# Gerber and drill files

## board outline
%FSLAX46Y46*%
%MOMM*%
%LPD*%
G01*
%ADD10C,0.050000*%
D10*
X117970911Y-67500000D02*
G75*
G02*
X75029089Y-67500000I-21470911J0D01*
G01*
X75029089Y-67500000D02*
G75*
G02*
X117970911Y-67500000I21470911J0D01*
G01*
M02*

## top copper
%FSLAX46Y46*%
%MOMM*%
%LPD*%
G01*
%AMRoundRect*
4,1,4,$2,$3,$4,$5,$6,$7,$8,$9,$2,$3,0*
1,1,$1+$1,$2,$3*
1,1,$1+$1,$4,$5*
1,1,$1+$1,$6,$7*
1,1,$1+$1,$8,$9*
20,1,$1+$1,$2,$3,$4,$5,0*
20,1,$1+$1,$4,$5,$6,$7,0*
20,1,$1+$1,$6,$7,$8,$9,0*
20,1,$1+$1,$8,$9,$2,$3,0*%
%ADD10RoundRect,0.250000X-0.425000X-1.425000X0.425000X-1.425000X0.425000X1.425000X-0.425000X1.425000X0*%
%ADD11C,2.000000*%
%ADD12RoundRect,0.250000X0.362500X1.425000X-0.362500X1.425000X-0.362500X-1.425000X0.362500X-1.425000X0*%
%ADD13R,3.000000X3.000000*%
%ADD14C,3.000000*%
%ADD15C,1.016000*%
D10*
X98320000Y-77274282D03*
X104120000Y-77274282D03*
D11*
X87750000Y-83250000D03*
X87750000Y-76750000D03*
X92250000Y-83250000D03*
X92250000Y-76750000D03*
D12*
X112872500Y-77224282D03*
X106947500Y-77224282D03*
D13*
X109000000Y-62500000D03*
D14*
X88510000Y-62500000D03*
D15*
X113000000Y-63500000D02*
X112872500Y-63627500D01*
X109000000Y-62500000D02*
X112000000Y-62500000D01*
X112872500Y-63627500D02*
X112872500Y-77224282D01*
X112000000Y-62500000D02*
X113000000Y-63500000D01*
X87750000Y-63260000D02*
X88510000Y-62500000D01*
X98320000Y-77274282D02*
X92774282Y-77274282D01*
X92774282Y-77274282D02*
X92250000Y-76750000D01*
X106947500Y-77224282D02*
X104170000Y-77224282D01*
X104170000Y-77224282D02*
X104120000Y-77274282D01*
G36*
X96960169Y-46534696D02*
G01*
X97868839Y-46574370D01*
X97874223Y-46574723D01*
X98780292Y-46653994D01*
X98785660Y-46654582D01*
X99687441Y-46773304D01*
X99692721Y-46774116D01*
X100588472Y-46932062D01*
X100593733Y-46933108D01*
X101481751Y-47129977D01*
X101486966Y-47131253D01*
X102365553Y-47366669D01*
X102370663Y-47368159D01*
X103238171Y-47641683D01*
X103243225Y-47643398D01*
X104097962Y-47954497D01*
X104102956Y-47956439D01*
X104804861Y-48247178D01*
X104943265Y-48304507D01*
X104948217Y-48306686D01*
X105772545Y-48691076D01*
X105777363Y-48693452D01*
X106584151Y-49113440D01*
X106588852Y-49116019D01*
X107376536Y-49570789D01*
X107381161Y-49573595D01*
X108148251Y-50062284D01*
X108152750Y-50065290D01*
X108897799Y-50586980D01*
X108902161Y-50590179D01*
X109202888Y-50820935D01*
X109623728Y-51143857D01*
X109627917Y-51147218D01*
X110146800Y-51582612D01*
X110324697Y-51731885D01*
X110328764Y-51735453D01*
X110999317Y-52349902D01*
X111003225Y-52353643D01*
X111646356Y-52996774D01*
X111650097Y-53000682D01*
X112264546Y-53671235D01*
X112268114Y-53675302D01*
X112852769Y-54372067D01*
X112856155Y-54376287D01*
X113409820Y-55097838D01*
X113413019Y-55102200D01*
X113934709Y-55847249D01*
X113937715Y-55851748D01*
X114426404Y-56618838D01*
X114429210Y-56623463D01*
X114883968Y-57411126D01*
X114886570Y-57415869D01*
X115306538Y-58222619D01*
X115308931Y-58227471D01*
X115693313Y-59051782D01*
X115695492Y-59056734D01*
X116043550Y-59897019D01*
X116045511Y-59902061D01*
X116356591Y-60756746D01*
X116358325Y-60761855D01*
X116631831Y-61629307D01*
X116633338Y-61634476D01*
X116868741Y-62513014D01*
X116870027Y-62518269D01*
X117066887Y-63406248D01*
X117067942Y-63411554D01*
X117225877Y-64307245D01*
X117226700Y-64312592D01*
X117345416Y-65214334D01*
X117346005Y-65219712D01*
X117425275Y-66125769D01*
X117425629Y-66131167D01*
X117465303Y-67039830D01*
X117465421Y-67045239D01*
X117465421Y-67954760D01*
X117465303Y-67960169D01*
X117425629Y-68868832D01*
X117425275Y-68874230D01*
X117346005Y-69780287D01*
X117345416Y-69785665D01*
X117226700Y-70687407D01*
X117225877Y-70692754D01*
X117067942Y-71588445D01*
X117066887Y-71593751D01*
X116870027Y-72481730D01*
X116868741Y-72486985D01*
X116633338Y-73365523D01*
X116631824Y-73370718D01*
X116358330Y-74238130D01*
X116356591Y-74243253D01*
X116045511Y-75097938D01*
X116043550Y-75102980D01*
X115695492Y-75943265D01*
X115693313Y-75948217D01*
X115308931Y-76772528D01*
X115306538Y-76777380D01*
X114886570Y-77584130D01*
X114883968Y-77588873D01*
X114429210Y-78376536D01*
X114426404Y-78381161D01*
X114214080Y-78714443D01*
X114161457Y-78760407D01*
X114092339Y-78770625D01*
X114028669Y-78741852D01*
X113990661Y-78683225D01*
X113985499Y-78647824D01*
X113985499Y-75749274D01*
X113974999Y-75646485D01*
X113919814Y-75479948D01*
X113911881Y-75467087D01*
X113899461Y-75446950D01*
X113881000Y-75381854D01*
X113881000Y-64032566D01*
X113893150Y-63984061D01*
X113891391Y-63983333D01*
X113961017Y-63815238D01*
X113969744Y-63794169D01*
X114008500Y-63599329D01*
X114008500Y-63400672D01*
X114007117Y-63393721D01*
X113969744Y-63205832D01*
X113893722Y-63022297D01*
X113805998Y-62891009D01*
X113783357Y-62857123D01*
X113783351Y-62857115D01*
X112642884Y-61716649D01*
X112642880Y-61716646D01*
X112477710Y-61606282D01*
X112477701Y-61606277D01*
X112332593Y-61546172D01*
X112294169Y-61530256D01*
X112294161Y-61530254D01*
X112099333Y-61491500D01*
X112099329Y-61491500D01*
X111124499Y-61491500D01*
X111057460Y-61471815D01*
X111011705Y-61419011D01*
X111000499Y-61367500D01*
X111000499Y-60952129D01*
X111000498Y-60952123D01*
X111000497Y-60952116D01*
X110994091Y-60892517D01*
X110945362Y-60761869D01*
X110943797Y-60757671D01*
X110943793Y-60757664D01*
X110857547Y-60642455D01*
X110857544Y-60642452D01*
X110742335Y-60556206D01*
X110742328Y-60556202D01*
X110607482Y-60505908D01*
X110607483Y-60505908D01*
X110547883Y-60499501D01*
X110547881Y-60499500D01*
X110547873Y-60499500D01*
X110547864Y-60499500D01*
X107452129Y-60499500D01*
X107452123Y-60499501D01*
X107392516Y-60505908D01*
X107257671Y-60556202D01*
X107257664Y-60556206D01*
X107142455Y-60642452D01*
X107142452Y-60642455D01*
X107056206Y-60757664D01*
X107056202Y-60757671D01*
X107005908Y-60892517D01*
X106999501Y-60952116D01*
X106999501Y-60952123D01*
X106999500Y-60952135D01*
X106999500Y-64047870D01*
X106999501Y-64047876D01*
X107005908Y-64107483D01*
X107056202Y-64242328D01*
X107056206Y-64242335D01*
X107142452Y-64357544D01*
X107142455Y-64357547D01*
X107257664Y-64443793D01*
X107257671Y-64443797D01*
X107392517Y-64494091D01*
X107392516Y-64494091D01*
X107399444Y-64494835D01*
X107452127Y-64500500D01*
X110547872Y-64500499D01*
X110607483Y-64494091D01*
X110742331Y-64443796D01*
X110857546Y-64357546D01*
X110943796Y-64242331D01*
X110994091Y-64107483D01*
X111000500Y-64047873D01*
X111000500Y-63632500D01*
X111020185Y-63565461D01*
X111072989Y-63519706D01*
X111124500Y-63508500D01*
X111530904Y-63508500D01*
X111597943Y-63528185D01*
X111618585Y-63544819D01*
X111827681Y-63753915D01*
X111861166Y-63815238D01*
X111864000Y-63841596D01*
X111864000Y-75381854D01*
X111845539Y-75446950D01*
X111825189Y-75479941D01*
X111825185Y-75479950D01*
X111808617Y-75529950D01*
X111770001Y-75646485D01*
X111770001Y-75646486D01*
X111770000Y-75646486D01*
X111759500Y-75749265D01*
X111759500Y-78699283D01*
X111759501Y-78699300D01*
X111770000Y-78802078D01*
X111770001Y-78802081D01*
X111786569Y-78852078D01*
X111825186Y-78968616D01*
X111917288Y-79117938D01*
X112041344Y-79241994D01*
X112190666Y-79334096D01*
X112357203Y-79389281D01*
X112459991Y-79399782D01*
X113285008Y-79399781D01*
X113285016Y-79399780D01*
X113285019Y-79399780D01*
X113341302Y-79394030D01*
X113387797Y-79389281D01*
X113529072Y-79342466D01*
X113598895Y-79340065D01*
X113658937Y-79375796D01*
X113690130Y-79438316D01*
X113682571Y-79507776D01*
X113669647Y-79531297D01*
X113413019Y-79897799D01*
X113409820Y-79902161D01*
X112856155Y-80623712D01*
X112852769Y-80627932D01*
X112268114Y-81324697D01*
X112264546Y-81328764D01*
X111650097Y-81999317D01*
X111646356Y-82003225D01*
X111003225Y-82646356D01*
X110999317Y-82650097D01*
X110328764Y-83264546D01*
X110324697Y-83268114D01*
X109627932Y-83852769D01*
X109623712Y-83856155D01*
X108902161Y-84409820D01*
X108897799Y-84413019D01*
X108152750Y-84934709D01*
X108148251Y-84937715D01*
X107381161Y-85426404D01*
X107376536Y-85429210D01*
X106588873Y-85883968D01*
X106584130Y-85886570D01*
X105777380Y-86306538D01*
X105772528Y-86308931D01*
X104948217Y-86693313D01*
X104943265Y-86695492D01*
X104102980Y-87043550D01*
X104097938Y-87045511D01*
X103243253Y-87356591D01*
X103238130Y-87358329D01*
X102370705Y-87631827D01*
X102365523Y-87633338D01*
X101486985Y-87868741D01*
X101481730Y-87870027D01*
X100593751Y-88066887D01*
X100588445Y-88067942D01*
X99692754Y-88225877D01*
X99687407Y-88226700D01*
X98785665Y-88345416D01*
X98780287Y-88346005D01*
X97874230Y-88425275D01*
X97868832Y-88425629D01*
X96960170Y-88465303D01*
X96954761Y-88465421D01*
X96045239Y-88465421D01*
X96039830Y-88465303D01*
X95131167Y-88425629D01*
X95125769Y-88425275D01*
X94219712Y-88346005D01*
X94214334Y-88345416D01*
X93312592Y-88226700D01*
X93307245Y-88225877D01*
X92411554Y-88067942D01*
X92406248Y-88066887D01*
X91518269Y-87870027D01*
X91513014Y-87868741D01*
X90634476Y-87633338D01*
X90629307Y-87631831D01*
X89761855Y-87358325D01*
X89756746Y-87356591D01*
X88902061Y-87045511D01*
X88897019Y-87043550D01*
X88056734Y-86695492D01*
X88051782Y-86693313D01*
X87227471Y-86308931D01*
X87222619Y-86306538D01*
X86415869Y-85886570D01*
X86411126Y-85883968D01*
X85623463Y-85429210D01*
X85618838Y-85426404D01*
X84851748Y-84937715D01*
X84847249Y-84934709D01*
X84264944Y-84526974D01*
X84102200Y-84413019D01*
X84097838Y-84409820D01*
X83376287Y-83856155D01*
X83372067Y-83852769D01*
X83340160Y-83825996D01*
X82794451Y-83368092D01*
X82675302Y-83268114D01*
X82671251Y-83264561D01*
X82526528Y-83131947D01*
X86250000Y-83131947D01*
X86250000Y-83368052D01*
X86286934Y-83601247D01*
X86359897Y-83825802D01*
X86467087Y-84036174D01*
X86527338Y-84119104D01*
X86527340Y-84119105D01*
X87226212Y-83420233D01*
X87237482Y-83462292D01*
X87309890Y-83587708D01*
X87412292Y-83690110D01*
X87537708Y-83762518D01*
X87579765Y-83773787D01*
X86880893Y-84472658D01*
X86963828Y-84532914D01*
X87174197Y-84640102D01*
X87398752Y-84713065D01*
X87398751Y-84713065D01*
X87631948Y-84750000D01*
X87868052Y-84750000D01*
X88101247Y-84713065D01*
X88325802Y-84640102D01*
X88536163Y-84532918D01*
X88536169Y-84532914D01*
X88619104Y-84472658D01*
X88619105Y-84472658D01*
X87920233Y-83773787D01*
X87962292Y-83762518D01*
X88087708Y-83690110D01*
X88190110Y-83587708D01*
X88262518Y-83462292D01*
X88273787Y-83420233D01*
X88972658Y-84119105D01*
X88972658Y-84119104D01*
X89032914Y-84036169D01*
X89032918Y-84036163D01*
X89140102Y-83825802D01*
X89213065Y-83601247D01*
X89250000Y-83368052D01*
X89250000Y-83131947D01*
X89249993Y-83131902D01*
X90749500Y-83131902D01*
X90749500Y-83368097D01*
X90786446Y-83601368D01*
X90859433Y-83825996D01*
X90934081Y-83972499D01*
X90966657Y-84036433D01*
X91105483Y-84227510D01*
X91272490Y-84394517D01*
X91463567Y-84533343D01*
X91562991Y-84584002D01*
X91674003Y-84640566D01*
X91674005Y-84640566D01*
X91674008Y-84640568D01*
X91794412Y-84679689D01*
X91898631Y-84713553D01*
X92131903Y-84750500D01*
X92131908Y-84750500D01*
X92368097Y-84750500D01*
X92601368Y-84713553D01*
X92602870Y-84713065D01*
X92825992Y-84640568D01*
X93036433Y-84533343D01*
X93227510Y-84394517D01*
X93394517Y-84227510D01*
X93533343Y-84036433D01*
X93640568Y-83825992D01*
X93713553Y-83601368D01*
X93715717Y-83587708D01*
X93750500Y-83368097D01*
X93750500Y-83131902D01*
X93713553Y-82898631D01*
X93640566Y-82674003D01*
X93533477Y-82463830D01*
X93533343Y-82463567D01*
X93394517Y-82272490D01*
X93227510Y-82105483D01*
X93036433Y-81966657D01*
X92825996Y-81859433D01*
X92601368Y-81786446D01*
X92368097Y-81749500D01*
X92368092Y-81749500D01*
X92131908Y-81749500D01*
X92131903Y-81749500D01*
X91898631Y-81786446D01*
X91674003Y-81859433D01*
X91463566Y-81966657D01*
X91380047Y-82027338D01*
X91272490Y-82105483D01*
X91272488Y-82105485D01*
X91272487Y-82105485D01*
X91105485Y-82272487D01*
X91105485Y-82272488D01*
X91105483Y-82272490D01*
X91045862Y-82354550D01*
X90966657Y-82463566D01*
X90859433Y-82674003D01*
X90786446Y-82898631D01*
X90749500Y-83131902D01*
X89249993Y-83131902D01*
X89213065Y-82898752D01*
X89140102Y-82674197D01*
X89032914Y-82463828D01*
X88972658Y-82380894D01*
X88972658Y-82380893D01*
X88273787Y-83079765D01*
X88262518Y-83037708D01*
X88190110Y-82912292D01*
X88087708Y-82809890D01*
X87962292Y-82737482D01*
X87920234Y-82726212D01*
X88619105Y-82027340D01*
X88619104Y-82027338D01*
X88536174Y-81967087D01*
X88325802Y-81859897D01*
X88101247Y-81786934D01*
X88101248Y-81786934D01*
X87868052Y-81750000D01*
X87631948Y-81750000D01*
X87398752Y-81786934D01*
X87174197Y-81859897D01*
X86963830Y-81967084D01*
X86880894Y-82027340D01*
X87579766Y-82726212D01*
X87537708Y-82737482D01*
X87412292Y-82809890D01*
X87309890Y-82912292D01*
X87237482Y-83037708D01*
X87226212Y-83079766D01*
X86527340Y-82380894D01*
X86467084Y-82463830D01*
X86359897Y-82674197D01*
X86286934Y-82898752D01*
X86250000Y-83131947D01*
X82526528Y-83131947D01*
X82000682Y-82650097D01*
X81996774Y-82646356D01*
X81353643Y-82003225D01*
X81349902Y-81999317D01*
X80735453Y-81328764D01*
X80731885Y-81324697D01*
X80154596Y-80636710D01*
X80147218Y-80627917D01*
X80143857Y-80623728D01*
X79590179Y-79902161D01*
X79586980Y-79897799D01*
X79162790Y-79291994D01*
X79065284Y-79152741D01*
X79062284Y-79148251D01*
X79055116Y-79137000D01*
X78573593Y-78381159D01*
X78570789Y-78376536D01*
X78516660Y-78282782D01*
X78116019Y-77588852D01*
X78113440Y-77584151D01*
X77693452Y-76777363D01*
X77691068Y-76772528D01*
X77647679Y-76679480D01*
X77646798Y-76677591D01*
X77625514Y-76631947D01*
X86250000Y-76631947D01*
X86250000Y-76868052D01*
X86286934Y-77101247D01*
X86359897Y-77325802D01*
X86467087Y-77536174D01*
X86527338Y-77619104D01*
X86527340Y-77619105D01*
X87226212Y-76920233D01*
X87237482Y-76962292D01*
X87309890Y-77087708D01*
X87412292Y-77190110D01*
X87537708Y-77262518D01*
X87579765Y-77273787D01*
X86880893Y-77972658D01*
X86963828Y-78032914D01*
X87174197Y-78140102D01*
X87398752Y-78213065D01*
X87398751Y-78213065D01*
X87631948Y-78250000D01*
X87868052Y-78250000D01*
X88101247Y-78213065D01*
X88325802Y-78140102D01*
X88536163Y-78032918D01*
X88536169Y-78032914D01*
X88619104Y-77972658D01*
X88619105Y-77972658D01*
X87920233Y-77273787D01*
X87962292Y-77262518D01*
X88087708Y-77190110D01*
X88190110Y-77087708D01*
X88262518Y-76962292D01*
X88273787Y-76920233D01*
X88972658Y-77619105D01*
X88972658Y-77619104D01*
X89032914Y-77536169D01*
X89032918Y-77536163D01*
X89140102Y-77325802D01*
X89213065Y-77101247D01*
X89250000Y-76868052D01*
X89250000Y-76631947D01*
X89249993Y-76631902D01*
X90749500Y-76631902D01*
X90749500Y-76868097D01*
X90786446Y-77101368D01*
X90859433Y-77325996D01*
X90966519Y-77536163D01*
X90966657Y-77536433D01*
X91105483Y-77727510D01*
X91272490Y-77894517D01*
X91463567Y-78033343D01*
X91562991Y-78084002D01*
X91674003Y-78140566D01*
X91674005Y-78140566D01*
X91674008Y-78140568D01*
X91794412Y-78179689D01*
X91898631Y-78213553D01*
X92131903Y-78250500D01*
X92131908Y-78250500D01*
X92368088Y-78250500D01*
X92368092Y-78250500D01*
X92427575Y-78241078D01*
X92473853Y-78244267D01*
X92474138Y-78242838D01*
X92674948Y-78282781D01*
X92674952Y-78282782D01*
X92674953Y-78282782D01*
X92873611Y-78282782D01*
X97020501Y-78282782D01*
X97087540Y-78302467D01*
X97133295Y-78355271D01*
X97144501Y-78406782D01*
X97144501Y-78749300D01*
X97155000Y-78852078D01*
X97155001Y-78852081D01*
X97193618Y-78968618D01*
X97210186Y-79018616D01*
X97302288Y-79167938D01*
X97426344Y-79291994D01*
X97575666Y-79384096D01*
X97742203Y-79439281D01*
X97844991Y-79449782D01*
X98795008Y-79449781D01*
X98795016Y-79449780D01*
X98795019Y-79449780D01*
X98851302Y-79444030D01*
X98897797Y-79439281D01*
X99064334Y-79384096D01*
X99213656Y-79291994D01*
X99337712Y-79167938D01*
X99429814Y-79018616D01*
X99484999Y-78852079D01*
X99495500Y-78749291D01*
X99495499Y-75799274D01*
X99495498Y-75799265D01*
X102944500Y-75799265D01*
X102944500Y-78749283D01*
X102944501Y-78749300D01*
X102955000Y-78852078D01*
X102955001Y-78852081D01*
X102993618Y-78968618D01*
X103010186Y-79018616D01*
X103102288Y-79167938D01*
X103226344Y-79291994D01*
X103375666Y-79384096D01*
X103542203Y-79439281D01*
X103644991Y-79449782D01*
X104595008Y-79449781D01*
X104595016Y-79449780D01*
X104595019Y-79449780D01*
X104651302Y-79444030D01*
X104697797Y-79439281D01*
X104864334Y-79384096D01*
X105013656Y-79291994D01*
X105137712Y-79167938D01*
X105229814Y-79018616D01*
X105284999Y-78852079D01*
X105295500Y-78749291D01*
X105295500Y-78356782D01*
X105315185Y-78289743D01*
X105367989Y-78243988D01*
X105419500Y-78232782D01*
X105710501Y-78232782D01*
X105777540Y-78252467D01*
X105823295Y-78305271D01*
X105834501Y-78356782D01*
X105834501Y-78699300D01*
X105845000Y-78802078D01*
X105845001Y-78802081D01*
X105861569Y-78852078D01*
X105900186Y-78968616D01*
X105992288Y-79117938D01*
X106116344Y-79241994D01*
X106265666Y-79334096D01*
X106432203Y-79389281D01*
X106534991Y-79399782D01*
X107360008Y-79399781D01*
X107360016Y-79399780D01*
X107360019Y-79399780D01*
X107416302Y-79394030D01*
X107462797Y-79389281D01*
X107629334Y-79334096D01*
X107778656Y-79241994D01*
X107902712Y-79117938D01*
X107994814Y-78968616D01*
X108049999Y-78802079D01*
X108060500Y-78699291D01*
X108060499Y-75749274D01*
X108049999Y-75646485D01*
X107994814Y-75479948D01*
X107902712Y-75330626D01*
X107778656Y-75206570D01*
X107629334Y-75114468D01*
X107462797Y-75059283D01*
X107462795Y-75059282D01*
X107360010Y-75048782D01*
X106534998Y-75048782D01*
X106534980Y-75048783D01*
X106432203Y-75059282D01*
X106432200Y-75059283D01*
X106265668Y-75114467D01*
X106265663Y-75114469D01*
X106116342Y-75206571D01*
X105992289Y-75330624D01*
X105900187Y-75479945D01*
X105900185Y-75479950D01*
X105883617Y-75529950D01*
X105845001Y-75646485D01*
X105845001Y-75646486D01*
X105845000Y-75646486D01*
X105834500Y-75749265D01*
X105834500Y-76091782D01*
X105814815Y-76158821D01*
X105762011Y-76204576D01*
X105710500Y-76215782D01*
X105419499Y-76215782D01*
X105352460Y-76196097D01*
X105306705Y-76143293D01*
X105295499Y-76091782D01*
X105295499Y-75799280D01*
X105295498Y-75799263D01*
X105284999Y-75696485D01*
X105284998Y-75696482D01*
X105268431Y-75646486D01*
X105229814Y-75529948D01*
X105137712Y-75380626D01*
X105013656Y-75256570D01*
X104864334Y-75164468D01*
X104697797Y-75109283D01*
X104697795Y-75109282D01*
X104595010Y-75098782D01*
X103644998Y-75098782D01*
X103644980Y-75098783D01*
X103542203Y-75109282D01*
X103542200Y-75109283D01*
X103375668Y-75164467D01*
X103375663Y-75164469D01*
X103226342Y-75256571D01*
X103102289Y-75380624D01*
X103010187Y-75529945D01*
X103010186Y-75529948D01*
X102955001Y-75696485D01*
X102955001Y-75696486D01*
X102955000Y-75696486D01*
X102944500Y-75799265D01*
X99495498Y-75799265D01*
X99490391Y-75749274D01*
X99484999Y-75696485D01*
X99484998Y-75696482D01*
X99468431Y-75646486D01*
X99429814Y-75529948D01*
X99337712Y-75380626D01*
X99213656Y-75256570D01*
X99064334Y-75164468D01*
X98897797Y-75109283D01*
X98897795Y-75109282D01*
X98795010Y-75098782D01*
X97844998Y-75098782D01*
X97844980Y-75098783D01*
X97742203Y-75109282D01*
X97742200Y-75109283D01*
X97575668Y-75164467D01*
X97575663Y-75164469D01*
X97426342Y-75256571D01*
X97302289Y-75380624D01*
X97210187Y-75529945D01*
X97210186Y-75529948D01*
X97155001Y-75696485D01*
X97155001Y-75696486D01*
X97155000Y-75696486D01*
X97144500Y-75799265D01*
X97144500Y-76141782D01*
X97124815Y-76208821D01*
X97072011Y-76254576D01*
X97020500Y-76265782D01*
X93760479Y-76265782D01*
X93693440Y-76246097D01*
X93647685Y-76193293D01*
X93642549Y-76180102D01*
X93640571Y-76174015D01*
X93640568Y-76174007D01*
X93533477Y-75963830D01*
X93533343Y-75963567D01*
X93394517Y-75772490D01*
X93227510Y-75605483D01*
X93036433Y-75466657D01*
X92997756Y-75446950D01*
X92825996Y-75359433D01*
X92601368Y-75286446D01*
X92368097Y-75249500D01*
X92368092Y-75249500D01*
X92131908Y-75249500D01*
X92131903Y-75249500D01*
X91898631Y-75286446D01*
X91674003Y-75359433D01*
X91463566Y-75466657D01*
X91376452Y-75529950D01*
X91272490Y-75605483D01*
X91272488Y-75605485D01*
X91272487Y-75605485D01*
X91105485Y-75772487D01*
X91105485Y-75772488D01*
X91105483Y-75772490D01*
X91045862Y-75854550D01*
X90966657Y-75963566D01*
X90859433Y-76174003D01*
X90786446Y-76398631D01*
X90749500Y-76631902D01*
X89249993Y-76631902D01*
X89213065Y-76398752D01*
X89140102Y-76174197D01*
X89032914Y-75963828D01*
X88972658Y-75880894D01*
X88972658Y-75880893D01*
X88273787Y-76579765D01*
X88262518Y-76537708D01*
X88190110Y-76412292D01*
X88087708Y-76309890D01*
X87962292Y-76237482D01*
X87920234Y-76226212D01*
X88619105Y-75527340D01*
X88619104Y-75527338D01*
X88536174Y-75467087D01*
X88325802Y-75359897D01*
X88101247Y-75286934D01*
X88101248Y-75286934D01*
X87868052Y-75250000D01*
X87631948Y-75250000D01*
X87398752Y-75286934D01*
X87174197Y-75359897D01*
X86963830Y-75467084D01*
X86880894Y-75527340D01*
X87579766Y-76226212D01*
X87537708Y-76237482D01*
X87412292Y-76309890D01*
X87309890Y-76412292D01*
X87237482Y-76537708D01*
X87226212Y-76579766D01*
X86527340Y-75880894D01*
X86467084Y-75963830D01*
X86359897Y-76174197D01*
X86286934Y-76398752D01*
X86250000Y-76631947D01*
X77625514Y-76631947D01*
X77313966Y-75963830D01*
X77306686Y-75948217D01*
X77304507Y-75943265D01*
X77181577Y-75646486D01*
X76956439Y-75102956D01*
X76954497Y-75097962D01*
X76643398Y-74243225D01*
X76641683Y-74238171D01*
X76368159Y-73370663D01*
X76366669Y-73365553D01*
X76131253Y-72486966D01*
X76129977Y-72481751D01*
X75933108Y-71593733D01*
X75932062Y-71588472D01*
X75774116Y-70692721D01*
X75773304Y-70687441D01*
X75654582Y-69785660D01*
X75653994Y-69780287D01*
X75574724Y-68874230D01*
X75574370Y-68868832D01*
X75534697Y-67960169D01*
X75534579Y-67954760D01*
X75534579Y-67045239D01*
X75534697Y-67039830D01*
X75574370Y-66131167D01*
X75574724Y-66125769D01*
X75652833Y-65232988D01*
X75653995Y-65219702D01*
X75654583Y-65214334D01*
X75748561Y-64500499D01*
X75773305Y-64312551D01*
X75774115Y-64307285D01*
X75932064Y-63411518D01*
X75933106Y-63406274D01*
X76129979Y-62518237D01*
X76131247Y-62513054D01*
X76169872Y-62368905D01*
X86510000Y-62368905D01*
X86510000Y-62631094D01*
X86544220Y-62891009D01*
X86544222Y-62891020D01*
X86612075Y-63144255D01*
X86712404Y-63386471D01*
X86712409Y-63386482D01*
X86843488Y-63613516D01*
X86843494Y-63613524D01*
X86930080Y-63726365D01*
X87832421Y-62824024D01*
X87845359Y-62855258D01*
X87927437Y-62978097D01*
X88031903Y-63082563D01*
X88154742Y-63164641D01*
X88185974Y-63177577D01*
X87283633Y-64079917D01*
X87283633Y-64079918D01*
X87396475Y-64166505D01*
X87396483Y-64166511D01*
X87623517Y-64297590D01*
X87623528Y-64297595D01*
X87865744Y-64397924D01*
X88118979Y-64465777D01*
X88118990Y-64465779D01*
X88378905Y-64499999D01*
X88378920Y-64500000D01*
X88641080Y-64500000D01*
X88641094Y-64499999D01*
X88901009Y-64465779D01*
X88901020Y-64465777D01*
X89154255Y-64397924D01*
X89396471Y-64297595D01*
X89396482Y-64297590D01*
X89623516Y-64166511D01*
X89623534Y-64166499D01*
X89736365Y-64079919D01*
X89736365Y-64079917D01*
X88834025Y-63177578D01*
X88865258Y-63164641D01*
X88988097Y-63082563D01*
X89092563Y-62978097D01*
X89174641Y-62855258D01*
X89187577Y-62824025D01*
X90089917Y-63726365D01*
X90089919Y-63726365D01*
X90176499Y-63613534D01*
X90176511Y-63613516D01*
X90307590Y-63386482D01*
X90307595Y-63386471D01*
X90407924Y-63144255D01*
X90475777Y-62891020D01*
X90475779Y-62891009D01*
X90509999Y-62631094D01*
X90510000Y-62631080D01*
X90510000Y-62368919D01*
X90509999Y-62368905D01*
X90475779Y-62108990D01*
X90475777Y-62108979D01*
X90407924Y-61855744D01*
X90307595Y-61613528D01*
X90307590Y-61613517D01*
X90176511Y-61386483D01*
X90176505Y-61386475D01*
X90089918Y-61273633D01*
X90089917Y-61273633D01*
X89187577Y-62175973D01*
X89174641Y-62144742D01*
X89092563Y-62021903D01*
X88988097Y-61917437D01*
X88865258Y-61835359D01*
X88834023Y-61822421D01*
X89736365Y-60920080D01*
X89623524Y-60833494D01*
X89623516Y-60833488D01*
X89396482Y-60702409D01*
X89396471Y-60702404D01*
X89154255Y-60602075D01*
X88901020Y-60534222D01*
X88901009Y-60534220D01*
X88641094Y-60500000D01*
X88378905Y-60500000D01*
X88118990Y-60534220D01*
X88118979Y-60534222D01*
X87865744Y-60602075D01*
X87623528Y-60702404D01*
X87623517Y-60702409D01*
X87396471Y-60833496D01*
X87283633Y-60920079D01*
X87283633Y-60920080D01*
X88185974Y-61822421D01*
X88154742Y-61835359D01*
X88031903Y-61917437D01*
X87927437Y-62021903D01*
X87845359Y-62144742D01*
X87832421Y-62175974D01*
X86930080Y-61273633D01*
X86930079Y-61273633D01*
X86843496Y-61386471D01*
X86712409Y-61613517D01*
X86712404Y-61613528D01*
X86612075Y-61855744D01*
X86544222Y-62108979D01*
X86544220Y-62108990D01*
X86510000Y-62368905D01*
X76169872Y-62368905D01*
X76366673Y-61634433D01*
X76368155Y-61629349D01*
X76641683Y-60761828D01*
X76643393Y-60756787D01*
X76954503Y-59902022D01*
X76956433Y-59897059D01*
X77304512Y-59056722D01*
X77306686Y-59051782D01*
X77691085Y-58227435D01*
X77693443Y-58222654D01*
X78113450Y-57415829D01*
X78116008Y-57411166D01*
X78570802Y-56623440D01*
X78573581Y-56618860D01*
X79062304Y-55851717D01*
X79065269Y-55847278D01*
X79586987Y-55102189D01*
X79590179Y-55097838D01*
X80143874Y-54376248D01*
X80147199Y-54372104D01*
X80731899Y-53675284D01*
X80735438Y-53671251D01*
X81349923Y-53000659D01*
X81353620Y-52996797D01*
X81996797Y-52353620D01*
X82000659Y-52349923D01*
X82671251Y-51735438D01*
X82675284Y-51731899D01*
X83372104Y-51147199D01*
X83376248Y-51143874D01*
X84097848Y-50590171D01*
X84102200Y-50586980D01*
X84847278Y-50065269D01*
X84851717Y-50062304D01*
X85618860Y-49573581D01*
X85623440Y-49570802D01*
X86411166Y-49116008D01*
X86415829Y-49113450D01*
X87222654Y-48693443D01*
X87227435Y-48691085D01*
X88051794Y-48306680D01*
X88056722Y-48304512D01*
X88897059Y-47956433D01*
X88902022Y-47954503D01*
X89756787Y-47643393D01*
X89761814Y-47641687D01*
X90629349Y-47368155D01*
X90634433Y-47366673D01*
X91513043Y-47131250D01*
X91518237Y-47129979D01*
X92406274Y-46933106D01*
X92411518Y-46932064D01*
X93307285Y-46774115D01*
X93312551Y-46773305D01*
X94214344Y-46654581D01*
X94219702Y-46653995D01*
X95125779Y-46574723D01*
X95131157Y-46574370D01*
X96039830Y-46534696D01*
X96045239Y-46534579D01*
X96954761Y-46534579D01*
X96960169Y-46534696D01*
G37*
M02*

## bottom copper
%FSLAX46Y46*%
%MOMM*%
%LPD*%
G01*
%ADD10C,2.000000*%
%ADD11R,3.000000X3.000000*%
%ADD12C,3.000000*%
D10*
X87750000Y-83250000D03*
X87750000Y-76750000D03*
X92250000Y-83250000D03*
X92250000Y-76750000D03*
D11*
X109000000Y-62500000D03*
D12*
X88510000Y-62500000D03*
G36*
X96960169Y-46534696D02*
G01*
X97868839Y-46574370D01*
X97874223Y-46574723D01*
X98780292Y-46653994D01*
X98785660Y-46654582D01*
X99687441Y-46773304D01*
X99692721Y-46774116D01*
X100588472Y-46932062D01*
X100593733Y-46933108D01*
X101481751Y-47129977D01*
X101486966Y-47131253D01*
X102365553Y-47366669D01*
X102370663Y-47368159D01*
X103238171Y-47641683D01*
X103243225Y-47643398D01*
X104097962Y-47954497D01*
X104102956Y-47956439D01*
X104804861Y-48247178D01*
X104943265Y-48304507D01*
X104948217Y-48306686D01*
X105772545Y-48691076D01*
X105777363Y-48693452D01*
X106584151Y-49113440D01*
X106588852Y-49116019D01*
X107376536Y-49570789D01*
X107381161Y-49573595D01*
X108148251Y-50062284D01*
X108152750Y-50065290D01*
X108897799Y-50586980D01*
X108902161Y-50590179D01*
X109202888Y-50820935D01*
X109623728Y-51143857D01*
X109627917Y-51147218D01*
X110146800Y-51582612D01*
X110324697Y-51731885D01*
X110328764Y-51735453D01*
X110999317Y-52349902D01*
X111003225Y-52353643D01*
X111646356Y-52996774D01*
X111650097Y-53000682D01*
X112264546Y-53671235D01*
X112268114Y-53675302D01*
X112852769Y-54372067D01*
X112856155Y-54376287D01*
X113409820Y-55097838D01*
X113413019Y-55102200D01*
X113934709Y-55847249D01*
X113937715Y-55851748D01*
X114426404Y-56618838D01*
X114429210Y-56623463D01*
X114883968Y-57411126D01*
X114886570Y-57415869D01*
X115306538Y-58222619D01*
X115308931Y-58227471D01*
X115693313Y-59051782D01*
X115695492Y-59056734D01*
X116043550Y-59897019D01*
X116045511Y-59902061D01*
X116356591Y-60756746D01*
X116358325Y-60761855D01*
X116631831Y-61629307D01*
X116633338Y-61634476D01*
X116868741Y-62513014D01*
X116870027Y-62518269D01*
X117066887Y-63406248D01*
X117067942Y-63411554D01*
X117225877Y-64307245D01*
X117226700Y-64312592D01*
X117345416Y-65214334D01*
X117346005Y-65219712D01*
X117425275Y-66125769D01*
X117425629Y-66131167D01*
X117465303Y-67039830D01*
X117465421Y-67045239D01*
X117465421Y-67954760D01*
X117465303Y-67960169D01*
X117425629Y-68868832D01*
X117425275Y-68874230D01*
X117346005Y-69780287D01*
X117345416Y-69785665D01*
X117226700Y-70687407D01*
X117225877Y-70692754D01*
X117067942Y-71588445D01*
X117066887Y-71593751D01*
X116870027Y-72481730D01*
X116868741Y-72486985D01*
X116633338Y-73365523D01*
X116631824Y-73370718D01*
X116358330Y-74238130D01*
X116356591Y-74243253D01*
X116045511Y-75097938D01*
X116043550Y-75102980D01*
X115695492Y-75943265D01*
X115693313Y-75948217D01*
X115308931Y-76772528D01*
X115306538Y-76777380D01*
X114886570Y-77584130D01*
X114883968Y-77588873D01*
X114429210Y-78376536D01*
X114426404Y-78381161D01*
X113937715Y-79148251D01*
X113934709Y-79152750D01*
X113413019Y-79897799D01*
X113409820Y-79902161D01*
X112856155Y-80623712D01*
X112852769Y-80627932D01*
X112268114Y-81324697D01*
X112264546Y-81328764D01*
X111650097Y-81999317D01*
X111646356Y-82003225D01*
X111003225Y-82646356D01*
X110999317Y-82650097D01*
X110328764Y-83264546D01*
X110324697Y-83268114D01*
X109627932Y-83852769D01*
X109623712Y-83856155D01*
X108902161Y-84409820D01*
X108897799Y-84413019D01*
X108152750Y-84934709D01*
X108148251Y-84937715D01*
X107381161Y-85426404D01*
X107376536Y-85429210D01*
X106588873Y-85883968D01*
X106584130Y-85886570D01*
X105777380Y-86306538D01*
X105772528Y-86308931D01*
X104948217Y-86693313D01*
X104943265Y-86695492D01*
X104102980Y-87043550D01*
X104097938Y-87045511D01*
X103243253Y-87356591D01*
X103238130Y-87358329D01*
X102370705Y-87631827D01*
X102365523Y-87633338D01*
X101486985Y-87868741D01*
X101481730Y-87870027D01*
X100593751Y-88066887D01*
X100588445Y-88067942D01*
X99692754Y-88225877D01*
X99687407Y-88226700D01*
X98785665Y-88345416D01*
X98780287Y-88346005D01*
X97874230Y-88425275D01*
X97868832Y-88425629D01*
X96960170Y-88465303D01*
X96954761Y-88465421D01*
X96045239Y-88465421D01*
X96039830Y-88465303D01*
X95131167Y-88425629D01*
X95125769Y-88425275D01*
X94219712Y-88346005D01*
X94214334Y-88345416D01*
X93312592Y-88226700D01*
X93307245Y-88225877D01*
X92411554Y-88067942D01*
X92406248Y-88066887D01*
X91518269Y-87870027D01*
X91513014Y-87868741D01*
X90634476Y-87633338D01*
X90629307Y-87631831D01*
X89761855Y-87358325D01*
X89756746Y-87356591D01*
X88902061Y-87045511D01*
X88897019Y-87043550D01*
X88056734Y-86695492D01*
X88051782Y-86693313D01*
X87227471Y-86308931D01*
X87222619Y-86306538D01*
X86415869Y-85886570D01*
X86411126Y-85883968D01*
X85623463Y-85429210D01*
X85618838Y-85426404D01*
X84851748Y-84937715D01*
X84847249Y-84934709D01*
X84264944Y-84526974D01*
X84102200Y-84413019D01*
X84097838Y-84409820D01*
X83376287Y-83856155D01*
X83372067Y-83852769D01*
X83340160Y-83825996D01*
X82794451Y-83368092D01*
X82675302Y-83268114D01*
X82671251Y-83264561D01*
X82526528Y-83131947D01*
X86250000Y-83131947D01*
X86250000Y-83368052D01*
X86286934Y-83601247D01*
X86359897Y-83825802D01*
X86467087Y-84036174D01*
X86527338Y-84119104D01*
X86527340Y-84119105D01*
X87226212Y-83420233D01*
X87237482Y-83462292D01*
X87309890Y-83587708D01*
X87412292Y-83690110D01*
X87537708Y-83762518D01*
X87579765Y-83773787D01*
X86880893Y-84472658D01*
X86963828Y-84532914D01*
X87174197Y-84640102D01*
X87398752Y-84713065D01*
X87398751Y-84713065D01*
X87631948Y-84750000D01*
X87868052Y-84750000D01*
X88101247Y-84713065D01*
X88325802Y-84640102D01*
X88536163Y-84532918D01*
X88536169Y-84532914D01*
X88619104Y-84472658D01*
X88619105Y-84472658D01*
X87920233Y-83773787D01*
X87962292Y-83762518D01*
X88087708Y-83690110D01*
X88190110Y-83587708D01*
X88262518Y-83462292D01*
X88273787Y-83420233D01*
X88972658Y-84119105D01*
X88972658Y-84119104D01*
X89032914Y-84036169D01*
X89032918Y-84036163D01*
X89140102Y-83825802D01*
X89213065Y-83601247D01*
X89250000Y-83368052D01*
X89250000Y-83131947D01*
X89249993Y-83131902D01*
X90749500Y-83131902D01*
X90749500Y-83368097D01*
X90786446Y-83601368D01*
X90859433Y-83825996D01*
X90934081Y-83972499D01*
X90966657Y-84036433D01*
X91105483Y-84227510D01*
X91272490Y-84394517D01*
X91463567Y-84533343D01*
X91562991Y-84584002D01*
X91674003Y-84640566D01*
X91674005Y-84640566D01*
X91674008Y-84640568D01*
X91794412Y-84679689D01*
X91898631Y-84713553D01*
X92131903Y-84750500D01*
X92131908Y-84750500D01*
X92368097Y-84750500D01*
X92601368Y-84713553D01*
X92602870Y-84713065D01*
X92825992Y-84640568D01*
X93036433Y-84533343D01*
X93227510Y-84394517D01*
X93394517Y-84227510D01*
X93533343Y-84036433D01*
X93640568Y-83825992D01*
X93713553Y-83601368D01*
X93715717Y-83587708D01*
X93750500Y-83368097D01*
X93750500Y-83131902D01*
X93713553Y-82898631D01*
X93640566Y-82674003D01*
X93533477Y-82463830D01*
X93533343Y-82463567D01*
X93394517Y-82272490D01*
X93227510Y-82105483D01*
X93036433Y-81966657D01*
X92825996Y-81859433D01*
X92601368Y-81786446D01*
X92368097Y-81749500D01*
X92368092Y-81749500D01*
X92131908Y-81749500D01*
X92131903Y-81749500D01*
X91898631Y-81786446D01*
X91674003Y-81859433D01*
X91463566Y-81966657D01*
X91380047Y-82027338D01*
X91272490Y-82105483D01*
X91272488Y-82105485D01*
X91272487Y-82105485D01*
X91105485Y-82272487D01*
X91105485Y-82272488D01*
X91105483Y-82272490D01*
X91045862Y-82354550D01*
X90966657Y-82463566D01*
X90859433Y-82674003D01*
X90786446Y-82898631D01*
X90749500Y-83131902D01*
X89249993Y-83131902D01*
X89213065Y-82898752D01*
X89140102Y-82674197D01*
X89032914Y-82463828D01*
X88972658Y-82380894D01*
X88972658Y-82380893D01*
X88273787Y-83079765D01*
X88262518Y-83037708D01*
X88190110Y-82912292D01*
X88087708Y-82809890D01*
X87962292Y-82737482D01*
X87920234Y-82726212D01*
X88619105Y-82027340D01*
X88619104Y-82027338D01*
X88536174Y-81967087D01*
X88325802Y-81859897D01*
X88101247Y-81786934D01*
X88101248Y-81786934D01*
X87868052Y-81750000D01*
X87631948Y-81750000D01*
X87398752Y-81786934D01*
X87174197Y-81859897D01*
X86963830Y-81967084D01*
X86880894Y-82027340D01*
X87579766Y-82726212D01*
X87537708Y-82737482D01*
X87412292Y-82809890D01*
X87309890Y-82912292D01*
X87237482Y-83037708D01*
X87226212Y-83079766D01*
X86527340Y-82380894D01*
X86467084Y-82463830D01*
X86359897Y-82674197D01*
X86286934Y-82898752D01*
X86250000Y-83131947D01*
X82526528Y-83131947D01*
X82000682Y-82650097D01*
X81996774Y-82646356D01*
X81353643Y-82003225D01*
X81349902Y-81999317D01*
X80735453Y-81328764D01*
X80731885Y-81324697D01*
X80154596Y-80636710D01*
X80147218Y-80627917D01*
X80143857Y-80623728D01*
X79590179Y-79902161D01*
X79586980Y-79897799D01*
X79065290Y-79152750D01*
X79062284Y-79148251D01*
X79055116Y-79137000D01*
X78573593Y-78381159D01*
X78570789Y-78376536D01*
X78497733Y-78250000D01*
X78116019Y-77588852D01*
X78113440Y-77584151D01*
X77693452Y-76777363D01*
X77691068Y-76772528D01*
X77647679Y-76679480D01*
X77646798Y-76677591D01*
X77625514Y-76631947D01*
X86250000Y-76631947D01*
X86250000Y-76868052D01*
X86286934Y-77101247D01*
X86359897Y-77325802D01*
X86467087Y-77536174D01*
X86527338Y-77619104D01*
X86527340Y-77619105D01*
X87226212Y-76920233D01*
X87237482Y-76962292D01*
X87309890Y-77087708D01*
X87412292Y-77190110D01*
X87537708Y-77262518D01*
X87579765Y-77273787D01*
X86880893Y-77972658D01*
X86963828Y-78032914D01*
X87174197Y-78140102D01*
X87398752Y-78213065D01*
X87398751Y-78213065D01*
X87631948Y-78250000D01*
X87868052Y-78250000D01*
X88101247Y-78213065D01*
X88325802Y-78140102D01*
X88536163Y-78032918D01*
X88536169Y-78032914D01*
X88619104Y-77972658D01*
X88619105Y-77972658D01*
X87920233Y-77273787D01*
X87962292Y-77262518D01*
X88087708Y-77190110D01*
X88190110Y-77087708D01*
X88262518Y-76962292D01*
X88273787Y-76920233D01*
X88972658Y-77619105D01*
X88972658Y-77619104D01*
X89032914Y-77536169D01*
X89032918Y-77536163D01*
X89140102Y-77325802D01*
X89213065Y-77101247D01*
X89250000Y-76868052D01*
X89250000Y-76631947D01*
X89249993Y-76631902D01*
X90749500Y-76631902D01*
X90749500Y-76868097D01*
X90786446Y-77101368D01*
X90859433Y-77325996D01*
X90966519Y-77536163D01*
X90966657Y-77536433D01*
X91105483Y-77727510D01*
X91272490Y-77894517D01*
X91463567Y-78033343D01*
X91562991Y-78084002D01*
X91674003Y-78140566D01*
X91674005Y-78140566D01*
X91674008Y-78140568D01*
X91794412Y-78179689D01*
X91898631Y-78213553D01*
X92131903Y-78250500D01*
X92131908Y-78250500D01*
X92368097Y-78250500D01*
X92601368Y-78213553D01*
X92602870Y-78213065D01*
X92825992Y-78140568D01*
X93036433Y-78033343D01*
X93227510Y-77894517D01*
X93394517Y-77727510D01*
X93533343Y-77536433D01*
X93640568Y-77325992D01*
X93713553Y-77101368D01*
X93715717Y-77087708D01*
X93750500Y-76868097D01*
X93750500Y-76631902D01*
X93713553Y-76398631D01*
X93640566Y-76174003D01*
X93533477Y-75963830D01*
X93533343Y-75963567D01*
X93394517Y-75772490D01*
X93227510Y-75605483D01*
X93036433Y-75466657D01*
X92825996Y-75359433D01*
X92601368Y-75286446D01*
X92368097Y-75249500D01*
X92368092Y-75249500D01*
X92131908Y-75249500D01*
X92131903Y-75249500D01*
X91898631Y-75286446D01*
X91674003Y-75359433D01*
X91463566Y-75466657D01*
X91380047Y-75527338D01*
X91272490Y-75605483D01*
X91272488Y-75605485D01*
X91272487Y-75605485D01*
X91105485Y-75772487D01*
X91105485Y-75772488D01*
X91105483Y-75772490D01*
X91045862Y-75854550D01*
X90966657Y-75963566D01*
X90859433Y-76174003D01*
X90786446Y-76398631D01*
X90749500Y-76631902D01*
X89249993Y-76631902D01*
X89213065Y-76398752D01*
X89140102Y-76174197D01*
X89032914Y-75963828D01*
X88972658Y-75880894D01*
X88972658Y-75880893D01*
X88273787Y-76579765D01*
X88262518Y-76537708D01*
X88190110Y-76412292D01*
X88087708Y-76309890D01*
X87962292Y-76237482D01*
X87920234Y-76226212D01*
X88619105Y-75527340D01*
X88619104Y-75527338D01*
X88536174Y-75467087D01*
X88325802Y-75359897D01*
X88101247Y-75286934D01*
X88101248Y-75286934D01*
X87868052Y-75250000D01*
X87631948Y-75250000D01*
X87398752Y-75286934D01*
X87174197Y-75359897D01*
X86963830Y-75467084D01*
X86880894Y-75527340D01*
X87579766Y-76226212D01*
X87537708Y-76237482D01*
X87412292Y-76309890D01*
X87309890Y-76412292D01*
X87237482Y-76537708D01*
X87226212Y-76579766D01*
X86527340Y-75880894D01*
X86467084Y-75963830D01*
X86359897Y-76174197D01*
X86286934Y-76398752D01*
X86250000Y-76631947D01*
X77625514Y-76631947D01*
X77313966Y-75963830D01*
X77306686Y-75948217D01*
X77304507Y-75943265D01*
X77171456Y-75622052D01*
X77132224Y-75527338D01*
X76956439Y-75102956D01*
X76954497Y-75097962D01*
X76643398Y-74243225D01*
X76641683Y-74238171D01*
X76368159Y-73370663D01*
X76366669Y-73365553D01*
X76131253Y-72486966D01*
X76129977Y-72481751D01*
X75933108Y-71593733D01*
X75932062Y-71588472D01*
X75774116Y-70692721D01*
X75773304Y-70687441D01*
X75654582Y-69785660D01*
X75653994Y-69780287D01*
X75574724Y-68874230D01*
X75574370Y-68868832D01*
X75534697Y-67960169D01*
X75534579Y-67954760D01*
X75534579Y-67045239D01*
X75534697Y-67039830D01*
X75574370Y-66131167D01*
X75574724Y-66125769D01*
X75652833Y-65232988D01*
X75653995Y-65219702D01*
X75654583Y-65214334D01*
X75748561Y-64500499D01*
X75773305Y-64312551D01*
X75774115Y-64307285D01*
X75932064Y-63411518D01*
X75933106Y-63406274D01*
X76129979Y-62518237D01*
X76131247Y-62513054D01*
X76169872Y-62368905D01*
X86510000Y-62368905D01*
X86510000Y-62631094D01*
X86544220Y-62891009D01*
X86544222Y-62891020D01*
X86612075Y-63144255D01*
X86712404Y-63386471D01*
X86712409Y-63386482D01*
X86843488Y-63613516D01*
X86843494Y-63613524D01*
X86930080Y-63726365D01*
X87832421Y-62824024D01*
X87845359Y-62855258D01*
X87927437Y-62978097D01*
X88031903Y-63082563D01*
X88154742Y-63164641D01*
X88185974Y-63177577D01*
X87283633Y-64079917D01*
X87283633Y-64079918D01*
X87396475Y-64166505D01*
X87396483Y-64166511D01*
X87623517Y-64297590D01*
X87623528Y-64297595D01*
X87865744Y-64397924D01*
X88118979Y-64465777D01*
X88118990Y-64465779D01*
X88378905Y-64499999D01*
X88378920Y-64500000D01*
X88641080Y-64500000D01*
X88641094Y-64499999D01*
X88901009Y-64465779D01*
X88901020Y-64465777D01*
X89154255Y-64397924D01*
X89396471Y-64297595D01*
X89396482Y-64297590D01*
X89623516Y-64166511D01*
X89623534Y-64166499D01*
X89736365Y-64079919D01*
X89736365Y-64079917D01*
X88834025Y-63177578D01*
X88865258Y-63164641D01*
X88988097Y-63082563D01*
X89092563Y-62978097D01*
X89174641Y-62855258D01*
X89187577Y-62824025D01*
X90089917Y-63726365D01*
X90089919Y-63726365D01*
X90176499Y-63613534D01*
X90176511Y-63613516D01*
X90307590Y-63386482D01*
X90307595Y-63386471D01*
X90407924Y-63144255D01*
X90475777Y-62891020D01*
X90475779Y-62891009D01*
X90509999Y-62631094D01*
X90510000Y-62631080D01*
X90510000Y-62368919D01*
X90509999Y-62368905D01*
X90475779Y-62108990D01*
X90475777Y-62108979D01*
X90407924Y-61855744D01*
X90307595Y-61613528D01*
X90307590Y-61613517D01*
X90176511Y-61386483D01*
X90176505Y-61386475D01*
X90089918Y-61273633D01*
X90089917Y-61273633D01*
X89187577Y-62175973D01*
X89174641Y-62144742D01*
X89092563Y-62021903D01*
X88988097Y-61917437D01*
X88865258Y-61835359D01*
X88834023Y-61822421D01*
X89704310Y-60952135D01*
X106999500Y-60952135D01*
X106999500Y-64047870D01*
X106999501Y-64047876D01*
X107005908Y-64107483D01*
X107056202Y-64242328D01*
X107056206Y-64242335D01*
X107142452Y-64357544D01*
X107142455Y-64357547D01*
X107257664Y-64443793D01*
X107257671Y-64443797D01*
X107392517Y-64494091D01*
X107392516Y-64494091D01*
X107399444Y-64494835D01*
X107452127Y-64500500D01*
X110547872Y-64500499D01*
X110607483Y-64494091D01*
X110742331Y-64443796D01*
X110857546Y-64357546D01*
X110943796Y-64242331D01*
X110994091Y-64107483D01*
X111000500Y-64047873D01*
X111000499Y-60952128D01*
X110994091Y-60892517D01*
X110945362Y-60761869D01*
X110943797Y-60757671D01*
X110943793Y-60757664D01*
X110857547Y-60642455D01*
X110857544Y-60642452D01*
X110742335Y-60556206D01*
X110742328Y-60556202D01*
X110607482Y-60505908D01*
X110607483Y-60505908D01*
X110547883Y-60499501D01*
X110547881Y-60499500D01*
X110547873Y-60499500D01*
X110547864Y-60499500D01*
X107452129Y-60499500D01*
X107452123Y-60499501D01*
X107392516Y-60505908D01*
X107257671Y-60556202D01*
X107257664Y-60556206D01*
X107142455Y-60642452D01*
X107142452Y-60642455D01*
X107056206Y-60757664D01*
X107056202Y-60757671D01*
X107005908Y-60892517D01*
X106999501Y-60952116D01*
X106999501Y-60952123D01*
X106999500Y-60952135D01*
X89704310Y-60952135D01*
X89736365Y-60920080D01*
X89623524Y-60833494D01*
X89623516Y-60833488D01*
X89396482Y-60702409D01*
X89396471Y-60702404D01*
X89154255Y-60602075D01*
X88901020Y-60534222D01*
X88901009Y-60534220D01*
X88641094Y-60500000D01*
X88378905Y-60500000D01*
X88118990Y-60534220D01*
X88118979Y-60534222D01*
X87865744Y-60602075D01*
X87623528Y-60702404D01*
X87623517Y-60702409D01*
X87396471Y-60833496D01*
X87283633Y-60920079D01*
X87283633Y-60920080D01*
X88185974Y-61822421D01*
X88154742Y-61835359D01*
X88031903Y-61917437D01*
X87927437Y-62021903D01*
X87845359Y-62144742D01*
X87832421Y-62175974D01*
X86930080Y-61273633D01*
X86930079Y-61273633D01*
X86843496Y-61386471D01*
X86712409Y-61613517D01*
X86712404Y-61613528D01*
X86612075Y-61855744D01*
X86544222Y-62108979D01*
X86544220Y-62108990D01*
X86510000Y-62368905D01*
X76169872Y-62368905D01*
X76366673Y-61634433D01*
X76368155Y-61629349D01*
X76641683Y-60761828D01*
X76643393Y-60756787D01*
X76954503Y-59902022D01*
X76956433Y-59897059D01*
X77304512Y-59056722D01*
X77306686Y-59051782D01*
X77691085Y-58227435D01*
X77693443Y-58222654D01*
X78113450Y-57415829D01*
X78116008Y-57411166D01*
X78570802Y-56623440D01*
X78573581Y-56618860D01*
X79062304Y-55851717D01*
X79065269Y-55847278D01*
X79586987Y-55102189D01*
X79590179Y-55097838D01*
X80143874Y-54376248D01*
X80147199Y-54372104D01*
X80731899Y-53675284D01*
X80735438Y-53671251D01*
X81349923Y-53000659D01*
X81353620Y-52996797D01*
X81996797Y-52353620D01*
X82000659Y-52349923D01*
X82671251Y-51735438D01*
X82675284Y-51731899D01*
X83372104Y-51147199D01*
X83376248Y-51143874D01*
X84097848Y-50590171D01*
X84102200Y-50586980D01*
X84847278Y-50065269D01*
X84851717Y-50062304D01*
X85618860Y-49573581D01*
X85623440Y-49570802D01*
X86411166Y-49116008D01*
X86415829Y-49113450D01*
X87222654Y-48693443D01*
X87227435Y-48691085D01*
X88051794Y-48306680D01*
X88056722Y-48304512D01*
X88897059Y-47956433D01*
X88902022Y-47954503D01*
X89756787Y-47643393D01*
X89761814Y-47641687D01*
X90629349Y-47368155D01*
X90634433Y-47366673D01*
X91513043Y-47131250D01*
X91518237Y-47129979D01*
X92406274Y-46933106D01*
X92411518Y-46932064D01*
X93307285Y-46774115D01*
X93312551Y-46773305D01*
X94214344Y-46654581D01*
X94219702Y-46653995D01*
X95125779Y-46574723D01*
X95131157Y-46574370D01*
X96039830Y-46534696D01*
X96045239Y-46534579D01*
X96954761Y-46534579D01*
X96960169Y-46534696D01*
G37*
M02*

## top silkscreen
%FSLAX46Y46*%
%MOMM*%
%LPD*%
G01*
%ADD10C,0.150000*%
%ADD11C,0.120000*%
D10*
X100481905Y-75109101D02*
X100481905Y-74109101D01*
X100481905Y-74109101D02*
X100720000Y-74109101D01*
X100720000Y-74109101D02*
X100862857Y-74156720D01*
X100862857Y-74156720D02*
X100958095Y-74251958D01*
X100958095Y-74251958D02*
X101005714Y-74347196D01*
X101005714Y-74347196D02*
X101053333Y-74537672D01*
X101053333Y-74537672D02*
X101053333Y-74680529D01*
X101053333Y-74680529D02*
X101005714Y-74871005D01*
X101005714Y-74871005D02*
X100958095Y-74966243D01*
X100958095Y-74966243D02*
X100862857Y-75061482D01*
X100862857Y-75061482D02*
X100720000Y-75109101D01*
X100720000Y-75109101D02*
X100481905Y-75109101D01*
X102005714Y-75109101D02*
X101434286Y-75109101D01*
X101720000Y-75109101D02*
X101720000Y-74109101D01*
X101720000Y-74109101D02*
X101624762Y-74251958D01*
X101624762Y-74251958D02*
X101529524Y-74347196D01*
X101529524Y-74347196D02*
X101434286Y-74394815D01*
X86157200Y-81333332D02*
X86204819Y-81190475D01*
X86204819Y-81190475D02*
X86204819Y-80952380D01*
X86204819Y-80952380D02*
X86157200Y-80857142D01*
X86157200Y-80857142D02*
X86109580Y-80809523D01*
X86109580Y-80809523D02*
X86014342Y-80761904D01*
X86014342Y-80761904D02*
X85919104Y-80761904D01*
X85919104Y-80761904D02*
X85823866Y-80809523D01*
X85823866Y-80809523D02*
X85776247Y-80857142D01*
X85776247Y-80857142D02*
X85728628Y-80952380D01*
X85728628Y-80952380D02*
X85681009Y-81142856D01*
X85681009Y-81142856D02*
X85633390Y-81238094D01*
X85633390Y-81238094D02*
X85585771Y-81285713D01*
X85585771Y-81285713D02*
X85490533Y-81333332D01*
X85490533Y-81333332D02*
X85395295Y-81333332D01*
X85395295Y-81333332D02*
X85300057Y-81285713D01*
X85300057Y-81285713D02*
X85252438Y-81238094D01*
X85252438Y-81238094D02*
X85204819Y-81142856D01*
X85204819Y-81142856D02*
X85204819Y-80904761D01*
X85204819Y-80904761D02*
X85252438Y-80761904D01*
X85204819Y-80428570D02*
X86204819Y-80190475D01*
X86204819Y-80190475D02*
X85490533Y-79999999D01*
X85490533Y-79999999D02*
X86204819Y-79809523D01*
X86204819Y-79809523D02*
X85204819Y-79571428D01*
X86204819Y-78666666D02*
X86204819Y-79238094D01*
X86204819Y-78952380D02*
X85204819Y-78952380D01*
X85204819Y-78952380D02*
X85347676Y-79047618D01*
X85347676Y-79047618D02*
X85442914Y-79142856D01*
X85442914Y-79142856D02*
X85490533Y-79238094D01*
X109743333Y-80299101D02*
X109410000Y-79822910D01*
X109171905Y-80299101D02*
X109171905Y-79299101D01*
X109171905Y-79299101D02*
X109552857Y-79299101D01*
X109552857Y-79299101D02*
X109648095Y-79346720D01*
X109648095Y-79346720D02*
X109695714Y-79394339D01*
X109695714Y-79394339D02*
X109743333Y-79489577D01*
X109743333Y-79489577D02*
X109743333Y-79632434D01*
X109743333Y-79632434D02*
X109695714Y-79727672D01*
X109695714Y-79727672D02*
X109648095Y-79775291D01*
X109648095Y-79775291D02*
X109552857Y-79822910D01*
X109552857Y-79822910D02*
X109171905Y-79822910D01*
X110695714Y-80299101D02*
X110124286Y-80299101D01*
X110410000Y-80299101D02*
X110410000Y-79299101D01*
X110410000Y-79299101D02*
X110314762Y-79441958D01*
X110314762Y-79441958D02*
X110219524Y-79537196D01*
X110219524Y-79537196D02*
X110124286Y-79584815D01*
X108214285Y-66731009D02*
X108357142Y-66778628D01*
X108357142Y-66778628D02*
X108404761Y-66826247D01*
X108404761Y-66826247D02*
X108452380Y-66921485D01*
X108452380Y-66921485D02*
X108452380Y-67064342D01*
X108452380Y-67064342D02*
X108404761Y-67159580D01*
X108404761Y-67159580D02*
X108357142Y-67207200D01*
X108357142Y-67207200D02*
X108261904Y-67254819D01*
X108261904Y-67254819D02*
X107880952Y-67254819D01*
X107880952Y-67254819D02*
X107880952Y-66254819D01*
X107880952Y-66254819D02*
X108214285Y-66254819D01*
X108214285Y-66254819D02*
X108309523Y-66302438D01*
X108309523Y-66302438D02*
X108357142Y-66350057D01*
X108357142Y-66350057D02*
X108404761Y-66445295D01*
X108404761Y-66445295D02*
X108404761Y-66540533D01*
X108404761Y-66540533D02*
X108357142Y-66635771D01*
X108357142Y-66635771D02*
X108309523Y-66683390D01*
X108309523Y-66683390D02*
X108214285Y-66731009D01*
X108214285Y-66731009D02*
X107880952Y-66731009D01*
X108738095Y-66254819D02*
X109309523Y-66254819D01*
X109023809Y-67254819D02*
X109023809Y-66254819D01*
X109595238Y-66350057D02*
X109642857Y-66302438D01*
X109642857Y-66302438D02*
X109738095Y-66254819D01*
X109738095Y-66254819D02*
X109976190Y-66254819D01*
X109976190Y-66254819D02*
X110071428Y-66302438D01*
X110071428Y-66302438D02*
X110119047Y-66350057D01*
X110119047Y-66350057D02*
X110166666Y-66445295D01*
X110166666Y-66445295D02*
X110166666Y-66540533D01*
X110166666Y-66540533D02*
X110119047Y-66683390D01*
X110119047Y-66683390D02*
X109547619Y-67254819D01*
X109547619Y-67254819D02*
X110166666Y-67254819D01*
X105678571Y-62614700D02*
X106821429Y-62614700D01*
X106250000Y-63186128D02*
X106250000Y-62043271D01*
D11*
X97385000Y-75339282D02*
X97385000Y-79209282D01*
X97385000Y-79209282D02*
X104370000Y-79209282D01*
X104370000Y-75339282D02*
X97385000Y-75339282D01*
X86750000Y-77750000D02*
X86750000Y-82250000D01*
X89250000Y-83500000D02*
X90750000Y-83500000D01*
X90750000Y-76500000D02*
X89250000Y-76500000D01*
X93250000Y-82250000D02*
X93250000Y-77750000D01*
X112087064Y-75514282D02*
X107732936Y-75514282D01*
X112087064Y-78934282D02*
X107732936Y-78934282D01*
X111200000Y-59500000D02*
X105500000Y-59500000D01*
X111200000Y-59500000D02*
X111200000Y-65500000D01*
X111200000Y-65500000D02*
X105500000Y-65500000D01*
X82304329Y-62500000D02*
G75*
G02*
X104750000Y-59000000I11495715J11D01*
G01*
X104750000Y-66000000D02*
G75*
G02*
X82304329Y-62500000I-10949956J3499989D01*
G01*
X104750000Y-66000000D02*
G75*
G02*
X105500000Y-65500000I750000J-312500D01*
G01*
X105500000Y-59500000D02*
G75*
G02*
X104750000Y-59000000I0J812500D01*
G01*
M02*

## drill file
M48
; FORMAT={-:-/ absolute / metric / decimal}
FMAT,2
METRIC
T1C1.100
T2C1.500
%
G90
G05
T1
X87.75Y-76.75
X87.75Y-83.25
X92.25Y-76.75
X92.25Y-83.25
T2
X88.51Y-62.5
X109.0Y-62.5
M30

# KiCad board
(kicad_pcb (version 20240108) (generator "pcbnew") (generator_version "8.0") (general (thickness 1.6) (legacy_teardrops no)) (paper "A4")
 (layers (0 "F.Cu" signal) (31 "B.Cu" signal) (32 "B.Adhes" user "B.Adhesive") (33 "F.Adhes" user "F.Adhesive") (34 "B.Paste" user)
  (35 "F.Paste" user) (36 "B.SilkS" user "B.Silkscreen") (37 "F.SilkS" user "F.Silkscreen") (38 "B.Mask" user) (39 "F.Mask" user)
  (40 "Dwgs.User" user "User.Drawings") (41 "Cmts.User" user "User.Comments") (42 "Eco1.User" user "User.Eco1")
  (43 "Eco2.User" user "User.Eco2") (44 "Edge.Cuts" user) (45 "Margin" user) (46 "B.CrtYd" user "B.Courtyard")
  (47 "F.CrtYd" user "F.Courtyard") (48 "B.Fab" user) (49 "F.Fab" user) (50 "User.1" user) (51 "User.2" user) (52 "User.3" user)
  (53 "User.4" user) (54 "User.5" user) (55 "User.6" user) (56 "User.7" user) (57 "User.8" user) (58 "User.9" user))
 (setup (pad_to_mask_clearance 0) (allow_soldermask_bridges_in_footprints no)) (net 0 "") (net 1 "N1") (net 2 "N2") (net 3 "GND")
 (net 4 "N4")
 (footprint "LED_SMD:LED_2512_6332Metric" (layer "F.Cu") (at 101.22 77.274282)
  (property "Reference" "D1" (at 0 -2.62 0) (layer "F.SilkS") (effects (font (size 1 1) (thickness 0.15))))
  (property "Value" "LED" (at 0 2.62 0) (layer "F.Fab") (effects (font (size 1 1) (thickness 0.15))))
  (fp_line (start -3.835 -1.935) (end -3.835 1.935) (stroke (width 0.12) (type solid)) (layer "F.SilkS"))
  (fp_line (start -3.835 1.935) (end 3.15 1.935) (stroke (width 0.12) (type solid)) (layer "F.SilkS"))
  (fp_line (start 3.15 -1.935) (end -3.835 -1.935) (stroke (width 0.12) (type solid)) (layer "F.SilkS"))
  (pad "1" smd roundrect (at -2.9 0) (size 1.35 3.35) (layers "F.Cu" "F.Paste" "F.Mask") (roundrect_rratio 0.185185) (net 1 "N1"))
  (pad "2" smd roundrect (at 2.9 0) (size 1.35 3.35) (layers "F.Cu" "F.Paste" "F.Mask") (roundrect_rratio 0.185185) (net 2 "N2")))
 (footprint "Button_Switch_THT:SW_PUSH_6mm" (layer "F.Cu") (at 87.75 83.25 90)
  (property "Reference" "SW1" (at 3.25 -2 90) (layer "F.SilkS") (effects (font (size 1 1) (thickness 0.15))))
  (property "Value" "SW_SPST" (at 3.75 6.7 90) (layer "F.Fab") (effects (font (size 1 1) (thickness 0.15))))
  (fp_line (start 5.5 -1) (end 1 -1) (stroke (width 0.12) (type solid)) (layer "F.SilkS"))
  (fp_line (start -0.25 1.5) (end -0.25 3) (stroke (width 0.12) (type solid)) (layer "F.SilkS"))
  (fp_line (start 6.75 3) (end 6.75 1.5) (stroke (width 0.12) (type solid)) (layer "F.SilkS"))
  (fp_line (start 1 5.5) (end 5.5 5.5) (stroke (width 0.12) (type solid)) (layer "F.SilkS"))
  (pad "1" thru_hole circle (at 0 0 180) (size 2 2) (drill 1.1) (layers "*.Cu" "*.Mask") (remove_unused_layers no) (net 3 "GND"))
  (pad "1" thru_hole circle (at 6.5 0 180) (size 2 2) (drill 1.1) (layers "*.Cu" "*.Mask") (remove_unused_layers no) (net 3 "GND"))
  (pad "2" thru_hole circle (at 0 4.5 180) (size 2 2) (drill 1.1) (layers "*.Cu" "*.Mask") (remove_unused_layers no) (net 1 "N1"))
  (pad "2" thru_hole circle (at 6.5 4.5 180) (size 2 2) (drill 1.1) (layers "*.Cu" "*.Mask") (remove_unused_layers no) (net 1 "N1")))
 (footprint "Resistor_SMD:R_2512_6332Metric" (layer "F.Cu") (at 109.91 77.224282 180)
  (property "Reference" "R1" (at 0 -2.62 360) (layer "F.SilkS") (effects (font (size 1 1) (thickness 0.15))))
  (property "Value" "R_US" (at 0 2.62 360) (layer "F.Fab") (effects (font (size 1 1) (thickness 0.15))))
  (fp_line (start -2.177064 1.71) (end 2.177064 1.71) (stroke (width 0.12) (type solid)) (layer "F.SilkS"))
  (fp_line (start -2.177064 -1.71) (end 2.177064 -1.71) (stroke (width 0.12) (type solid)) (layer "F.SilkS"))
  (pad "1" smd roundrect (at -2.9625 0 180) (size 1.225 3.35) (layers "F.Cu" "F.Paste" "F.Mask") (roundrect_rratio 0.204082) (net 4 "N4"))
  (pad "2" smd roundrect (at 2.9625 0 180) (size 1.225 3.35) (layers "F.Cu" "F.Paste" "F.Mask") (roundrect_rratio 0.204082) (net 2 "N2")))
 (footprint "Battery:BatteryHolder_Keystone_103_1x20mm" (layer "F.Cu") (at 109 62.5 180)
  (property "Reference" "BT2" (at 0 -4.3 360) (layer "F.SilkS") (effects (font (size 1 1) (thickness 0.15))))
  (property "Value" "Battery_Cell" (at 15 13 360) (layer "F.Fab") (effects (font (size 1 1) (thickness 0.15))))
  (fp_line (start -2.2 3) (end 3.5 3) (stroke (width 0.12) (type solid)) (layer "F.SilkS"))
  (fp_line (start -2.2 3) (end -2.2 -3) (stroke (width 0.12) (type solid)) (layer "F.SilkS"))
  (fp_line (start -2.2 -3) (end 3.5 -3) (stroke (width 0.12) (type solid)) (layer "F.SilkS"))
  (fp_arc (start 26.695671 0) (mid 16.971103 11.358466) (end 4.25 3.5) (stroke (width 0.12) (type solid)) (layer "F.SilkS"))
  (fp_arc (start 4.25 -3.5) (mid 16.971103 -11.358466) (end 26.695671 0) (stroke (width 0.12) (type solid)) (layer "F.SilkS"))
  (fp_arc (start 4.25 -3.5) (mid 3.950694 -3.136459) (end 3.5 -3) (stroke (width 0.12) (type solid)) (layer "F.SilkS"))
  (fp_arc (start 3.5 3) (mid 3.950694 3.136459) (end 4.25 3.5) (stroke (width 0.12) (type solid)) (layer "F.SilkS"))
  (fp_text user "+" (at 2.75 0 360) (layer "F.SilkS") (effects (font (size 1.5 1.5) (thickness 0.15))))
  (pad "1" thru_hole rect (at 0 0 180) (size 3 3) (drill 1.5) (layers "*.Cu" "*.Mask") (remove_unused_layers no) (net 4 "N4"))
  (pad "2" thru_hole circle (at 20.49 0 180) (size 3 3) (drill 1.5) (layers "*.Cu" "*.Mask") (remove_unused_layers no) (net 3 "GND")))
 (gr_circle (center 96.5 67.5) (end 77.5 57.5) (stroke (width 0.05) (type default)) (fill none) (layer "Edge.Cuts"))
 (segment (start 113 63.5) (end 112.8725 63.6275) (width 1.016) (layer "F.Cu") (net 4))
 (segment (start 109 62.5) (end 112 62.5) (width 1.016) (layer "F.Cu") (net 4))
 (segment (start 112.8725 63.6275) (end 112.8725 77.224282) (width 1.016) (layer "F.Cu") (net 4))
 (segment (start 112 62.5) (end 113 63.5) (width 1.016) (layer "F.Cu") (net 4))
 (segment (start 87.75 63.26) (end 88.51 62.5) (width 1.016) (layer "F.Cu") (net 3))
 (segment (start 98.32 77.274282) (end 92.774282 77.274282) (width 1.016) (layer "F.Cu") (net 1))
 (segment (start 92.774282 77.274282) (end 92.25 76.75) (width 1.016) (layer "F.Cu") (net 1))
 (segment (start 106.9475 77.224282) (end 104.17 77.224282) (width 1.016) (layer "F.Cu") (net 2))
 (segment (start 104.17 77.224282) (end 104.12 77.274282) (width 1.016) (layer "F.Cu") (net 2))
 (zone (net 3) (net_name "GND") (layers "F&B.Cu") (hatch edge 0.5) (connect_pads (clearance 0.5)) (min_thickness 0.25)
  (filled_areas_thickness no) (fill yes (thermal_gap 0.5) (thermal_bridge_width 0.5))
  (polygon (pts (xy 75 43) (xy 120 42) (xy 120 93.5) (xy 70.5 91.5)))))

